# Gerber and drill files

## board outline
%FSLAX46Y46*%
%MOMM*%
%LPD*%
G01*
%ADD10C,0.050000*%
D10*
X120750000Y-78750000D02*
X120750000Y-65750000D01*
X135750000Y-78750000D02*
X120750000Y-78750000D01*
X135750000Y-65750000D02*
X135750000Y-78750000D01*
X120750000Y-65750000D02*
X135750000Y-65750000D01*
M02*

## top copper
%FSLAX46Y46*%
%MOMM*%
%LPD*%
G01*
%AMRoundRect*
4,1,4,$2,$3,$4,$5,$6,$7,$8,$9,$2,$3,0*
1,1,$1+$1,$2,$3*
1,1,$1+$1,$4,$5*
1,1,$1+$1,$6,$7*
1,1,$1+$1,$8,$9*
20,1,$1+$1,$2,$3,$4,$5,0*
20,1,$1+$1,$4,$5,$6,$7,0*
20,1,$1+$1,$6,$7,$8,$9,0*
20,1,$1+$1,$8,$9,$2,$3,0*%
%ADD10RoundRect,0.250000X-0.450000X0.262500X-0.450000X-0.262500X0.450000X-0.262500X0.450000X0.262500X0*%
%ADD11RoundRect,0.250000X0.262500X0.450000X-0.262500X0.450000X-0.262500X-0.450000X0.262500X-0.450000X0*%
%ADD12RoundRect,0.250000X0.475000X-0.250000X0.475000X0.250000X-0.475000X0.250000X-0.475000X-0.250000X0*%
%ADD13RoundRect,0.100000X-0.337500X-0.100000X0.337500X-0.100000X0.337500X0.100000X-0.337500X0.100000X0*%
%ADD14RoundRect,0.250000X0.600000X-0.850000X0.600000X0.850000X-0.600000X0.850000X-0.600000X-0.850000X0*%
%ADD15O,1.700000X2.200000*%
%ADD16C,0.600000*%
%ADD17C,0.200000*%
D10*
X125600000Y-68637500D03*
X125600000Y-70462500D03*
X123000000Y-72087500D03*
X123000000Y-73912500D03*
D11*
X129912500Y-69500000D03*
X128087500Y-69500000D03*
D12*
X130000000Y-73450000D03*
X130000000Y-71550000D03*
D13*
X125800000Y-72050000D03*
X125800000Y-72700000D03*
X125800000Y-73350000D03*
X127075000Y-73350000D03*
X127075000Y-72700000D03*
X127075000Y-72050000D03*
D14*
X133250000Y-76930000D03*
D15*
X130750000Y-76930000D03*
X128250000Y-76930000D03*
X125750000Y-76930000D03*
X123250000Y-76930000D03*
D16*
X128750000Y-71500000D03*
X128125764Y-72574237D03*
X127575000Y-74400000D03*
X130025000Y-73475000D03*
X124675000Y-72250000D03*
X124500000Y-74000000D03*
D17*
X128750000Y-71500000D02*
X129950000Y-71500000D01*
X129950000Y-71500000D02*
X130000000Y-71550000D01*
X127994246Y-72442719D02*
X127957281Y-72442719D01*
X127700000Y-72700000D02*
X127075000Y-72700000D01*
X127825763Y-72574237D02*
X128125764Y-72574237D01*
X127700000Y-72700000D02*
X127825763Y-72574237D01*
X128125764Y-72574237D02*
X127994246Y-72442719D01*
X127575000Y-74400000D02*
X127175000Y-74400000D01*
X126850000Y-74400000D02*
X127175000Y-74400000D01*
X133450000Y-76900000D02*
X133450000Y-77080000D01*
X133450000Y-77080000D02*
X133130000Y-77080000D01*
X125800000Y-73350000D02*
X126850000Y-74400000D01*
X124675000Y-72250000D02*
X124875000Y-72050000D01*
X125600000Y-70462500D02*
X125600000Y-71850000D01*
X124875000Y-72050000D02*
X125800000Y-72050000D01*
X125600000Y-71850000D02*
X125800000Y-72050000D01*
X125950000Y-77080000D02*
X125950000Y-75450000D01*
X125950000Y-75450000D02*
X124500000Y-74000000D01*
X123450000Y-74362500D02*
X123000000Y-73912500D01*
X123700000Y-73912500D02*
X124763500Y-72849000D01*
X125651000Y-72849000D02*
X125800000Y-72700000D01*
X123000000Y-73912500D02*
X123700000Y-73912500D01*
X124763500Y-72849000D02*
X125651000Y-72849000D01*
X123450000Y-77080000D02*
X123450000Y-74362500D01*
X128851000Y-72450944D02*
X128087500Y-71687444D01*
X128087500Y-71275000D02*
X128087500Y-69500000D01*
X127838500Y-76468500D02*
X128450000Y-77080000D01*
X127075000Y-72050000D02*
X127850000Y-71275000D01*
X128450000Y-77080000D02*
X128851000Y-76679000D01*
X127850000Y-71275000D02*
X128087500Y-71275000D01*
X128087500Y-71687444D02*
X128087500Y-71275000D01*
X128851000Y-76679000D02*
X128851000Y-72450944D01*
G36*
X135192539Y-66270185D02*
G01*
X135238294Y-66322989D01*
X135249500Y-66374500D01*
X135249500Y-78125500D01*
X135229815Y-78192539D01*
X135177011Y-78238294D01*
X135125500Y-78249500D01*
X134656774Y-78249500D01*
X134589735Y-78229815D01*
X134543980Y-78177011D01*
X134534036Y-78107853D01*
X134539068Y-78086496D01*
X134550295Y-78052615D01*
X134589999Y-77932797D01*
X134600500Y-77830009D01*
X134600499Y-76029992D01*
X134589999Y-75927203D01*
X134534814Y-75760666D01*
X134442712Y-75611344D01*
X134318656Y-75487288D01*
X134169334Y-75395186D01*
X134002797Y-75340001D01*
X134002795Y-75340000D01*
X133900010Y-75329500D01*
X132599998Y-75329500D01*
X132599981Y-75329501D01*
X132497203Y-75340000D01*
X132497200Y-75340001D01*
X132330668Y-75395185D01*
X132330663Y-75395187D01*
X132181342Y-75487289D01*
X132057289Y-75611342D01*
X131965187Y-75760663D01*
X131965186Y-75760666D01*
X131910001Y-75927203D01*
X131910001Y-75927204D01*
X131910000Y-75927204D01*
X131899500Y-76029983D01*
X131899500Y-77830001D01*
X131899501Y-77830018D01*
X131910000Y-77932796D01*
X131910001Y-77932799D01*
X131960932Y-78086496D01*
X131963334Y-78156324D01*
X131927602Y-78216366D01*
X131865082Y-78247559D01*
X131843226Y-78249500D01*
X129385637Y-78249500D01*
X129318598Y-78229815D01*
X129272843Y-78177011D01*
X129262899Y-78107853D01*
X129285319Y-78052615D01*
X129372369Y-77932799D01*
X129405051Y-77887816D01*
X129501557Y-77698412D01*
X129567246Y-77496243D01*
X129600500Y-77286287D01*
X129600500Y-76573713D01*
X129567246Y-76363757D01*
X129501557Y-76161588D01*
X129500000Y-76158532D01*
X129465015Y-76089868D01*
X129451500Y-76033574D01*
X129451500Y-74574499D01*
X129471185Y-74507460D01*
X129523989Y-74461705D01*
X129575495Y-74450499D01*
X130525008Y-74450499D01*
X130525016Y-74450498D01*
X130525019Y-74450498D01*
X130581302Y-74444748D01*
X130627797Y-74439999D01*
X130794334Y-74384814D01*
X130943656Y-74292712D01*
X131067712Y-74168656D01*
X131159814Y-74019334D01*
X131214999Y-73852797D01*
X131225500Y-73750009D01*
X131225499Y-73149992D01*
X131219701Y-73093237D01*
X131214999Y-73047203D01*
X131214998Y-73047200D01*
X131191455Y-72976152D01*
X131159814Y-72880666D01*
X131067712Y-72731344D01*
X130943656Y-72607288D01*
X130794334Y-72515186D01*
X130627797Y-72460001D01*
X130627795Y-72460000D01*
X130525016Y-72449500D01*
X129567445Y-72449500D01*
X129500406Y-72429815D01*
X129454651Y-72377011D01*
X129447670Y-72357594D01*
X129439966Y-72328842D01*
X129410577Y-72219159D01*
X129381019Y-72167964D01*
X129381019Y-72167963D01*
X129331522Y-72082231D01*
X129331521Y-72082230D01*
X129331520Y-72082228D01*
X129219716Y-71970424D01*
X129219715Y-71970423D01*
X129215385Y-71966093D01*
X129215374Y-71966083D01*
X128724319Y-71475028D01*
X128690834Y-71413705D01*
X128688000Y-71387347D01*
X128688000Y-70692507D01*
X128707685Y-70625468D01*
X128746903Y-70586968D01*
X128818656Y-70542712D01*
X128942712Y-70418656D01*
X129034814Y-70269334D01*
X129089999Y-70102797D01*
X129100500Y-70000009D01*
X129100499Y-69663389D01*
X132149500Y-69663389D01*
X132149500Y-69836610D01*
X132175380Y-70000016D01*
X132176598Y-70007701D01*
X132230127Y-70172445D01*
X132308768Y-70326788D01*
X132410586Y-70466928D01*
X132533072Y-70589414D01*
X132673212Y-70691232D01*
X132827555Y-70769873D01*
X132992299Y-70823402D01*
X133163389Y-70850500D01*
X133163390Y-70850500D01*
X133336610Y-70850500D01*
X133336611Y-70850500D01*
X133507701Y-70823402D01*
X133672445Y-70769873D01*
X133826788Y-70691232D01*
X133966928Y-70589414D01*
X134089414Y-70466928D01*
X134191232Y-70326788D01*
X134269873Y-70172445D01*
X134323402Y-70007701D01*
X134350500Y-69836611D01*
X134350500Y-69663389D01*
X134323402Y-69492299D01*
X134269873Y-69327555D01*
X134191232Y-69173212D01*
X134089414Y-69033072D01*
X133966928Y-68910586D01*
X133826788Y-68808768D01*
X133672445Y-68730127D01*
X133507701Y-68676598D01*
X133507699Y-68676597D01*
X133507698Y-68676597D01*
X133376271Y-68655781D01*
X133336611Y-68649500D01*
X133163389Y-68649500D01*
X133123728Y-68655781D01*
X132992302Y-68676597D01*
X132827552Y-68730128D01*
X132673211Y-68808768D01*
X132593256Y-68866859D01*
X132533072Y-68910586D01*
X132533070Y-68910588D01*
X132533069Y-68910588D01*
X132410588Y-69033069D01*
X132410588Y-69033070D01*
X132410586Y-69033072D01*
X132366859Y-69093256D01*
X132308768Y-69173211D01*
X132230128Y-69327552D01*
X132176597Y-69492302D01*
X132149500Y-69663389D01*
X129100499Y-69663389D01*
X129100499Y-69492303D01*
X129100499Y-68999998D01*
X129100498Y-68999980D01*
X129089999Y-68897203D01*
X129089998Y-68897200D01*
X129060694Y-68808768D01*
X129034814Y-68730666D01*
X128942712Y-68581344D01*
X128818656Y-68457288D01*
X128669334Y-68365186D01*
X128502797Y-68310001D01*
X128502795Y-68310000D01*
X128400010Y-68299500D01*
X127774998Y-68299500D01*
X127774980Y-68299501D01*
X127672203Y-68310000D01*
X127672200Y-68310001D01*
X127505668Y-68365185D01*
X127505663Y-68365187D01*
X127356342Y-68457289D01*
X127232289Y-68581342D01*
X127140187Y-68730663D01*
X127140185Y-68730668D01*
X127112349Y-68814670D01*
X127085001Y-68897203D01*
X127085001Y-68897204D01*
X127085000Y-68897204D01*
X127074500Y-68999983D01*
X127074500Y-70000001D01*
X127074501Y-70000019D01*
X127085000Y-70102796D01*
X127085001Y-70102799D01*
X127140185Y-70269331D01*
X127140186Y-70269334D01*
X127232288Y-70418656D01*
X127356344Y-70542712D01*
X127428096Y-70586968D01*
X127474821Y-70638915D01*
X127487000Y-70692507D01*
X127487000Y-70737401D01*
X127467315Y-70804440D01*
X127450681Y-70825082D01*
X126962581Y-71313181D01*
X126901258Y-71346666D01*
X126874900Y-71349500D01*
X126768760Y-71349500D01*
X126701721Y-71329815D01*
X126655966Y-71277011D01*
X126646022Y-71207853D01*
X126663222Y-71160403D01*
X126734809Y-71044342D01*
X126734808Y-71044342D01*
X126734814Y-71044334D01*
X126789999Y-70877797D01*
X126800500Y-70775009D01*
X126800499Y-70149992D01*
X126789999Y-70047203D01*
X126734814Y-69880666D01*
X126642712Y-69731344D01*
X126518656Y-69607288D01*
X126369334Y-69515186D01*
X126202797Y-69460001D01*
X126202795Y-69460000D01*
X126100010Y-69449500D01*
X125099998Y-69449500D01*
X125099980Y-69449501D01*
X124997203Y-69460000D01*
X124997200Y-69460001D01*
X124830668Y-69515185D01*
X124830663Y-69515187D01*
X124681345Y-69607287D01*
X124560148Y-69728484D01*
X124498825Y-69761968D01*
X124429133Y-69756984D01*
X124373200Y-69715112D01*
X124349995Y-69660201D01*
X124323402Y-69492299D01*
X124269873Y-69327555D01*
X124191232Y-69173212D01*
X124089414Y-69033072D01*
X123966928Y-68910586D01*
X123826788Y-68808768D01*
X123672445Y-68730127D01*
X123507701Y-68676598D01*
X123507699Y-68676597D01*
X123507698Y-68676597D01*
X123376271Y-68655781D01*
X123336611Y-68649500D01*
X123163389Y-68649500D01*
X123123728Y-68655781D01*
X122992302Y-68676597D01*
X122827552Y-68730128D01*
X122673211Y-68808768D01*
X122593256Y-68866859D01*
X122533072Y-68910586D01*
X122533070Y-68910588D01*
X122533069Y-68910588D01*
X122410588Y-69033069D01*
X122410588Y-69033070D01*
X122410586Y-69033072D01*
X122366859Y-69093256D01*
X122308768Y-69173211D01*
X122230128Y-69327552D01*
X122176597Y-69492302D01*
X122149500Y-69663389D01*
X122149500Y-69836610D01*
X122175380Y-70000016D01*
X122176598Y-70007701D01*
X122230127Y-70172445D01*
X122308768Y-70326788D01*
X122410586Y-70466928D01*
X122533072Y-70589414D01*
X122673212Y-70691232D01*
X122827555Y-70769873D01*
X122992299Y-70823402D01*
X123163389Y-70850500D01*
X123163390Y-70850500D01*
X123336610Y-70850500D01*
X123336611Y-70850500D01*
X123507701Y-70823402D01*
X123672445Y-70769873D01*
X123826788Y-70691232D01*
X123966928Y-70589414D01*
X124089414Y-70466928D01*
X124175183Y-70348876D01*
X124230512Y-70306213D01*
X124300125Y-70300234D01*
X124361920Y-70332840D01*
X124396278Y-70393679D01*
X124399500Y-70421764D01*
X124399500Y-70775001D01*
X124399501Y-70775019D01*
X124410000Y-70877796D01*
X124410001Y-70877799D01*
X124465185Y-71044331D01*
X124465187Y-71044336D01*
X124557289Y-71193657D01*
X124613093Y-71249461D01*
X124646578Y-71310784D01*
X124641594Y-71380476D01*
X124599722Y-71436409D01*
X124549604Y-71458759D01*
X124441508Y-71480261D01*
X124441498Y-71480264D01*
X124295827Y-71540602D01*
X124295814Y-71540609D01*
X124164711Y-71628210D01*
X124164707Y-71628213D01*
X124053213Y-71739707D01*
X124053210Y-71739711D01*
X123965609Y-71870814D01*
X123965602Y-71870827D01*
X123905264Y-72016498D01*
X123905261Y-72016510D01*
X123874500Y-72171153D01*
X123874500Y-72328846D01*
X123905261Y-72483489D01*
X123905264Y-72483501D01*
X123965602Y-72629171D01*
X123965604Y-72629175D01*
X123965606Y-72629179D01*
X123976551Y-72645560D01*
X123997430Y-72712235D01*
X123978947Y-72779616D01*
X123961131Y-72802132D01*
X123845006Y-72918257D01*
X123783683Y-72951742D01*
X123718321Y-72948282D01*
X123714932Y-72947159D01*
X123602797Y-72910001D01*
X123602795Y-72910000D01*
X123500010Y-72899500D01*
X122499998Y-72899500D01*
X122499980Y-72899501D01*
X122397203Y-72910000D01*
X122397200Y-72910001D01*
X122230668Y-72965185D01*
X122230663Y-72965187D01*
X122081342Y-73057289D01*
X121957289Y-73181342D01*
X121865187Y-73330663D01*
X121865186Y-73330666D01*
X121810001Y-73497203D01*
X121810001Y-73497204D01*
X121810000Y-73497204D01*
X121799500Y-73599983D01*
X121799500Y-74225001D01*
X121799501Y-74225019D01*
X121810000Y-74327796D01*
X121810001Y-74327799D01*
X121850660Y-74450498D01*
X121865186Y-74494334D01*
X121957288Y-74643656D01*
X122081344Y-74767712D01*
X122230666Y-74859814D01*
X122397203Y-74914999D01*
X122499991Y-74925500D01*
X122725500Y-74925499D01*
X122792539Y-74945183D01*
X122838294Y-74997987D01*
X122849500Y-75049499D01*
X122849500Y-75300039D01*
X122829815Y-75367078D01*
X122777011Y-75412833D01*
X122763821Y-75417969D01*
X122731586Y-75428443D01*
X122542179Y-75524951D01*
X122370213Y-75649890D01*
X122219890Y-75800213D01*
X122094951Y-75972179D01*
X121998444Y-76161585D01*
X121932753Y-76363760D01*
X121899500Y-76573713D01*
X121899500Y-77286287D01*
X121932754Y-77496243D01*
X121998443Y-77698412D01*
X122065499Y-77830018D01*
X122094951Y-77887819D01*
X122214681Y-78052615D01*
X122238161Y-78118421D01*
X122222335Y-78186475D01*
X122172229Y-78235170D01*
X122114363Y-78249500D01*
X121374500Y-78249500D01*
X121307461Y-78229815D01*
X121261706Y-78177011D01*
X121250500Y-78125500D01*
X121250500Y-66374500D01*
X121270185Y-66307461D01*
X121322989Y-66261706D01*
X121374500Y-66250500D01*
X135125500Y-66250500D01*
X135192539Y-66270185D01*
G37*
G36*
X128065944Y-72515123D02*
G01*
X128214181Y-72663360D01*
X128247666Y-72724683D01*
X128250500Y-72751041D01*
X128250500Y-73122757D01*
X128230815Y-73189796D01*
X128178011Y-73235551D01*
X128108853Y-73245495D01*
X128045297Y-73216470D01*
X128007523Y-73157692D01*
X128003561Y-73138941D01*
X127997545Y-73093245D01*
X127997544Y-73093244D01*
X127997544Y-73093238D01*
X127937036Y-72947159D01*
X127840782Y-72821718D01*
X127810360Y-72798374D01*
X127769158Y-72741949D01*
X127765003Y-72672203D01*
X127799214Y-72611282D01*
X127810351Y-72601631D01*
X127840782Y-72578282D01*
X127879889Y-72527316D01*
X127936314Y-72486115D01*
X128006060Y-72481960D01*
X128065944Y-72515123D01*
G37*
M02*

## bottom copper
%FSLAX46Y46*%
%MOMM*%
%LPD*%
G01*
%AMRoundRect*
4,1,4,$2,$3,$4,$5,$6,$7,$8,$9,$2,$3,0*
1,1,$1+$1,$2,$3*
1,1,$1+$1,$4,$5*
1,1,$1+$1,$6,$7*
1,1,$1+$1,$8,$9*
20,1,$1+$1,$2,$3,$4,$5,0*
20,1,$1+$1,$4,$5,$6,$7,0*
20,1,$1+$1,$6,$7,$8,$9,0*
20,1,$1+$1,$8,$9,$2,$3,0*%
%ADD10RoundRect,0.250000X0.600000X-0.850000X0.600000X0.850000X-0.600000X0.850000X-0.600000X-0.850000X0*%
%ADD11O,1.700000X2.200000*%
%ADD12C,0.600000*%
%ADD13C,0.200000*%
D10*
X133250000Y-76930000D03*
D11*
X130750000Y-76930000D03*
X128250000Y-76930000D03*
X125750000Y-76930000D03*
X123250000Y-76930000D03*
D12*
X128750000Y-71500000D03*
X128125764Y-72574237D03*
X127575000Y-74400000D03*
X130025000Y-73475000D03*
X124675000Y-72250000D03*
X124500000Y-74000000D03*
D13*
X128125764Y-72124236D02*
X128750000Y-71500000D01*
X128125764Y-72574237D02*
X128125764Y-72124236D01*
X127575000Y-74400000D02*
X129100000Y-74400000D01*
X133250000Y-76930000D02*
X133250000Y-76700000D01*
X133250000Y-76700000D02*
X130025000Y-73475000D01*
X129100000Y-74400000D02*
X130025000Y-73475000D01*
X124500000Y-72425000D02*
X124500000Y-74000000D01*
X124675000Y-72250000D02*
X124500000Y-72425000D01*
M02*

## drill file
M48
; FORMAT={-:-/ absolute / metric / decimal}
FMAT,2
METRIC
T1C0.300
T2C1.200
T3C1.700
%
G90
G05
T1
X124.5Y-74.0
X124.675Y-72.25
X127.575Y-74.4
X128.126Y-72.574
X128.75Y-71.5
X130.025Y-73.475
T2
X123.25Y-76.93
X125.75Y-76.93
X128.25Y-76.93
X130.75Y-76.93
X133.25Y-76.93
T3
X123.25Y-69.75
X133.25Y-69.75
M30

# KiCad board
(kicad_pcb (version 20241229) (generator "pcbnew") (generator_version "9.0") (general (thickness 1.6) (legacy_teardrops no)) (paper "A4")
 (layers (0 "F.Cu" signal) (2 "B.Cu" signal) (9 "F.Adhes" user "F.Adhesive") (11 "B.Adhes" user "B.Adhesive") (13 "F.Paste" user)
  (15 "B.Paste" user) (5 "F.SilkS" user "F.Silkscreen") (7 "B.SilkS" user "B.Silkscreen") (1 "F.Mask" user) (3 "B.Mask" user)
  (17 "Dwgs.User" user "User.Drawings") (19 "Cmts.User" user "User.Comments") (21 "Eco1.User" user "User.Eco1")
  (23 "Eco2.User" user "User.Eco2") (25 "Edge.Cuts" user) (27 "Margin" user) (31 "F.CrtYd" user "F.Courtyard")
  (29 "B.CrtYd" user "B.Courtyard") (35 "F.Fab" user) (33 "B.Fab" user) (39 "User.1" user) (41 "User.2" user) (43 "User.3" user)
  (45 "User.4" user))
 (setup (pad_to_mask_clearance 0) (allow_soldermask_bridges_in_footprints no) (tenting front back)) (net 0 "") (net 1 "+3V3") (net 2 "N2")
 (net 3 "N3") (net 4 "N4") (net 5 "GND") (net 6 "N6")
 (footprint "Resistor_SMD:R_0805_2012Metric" (layer "F.Cu") (at 125.6 69.55 -90)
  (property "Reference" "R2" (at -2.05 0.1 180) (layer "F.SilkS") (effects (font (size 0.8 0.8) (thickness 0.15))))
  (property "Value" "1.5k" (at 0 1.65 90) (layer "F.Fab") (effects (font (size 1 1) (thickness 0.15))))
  (pad "1" smd roundrect (at -0.9125 0 270) (size 1.025 1.4) (layers "F.Cu" "F.Mask" "F.Paste") (roundrect_rratio 0.243902) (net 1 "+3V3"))
  (pad "2" smd roundrect (at 0.9125 0 270) (size 1.025 1.4) (layers "F.Cu" "F.Mask" "F.Paste") (roundrect_rratio 0.243902) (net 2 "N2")))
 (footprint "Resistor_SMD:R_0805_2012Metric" (layer "F.Cu") (at 123 73 -90)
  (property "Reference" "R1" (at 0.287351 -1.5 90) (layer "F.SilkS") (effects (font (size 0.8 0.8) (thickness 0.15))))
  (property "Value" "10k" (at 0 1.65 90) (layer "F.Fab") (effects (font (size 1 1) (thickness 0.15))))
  (pad "1" smd roundrect (at -0.9125 0 270) (size 1.025 1.4) (layers "F.Cu" "F.Mask" "F.Paste") (roundrect_rratio 0.243902) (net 1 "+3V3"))
  (pad "2" smd roundrect (at 0.9125 0 270) (size 1.025 1.4) (layers "F.Cu" "F.Mask" "F.Paste") (roundrect_rratio 0.243902) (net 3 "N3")))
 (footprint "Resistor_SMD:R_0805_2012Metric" (layer "F.Cu") (at 129 69.5 180)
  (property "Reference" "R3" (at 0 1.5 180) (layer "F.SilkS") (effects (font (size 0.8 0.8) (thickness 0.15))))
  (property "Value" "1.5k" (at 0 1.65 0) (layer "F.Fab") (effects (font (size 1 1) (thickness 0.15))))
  (pad "1" smd roundrect (at -0.9125 0 180) (size 1.025 1.4) (layers "F.Cu" "F.Mask" "F.Paste") (roundrect_rratio 0.243902) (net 1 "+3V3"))
  (pad "2" smd roundrect (at 0.9125 0 180) (size 1.025 1.4) (layers "F.Cu" "F.Mask" "F.Paste") (roundrect_rratio 0.243902) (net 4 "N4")))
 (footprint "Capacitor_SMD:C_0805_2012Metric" (layer "F.Cu") (at 130 72.5 90)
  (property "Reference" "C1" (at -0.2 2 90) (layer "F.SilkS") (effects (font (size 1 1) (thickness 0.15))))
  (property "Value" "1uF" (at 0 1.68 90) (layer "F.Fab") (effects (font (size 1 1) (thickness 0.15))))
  (pad "1" smd roundrect (at -0.95 0 90) (size 1 1.45) (layers "F.Cu" "F.Mask" "F.Paste") (roundrect_rratio 0.25) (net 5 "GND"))
  (pad "2" smd roundrect (at 0.95 0 90) (size 1 1.45) (layers "F.Cu" "F.Mask" "F.Paste") (roundrect_rratio 0.25) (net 1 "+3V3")))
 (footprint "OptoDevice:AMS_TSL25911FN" (layer "F.Cu") (at 126.4375 72.7)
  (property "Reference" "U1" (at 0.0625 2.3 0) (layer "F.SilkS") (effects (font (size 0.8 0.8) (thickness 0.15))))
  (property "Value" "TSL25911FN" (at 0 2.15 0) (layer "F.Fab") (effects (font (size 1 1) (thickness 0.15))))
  (pad "1" smd roundrect (at -0.6375 -0.65) (size 0.875 0.4) (layers "F.Cu" "F.Mask" "F.Paste") (roundrect_rratio 0.25) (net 2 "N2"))
  (pad "2" smd roundrect (at -0.6375 0) (size 0.875 0.4) (layers "F.Cu" "F.Mask" "F.Paste") (roundrect_rratio 0.25) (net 3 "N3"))
  (pad "3" smd roundrect (at -0.6375 0.65) (size 0.875 0.4) (layers "F.Cu" "F.Mask" "F.Paste") (roundrect_rratio 0.25) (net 5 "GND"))
  (pad "4" smd roundrect (at 0.6375 0.65) (size 0.875 0.4) (layers "F.Cu" "F.Mask" "F.Paste") (roundrect_rratio 0.25) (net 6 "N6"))
  (pad "5" smd roundrect (at 0.6375 0) (size 0.875 0.4) (layers "F.Cu" "F.Mask" "F.Paste") (roundrect_rratio 0.25) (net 1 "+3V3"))
  (pad "6" smd roundrect (at 0.6375 -0.65) (size 0.875 0.4) (layers "F.Cu" "F.Mask" "F.Paste") (roundrect_rratio 0.25) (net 4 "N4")))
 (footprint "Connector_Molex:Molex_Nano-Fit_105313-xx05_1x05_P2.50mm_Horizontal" (layer "B.Cu") (at 133.25 76.93 90)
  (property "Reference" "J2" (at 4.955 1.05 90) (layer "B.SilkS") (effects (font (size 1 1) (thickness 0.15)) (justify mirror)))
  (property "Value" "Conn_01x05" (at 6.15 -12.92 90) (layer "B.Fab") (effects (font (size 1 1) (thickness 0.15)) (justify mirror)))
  (pad "" np_thru_hole circle (at 7.18 -10 90) (size 1.7 1.7) (drill 1.7) (layers "*.Cu" "*.Mask"))
  (pad "" np_thru_hole circle (at 7.18 0 90) (size 1.7 1.7) (drill 1.7) (layers "*.Cu" "*.Mask"))
  (pad "1" thru_hole roundrect (at 0 0 90) (size 2.2 1.7) (drill 1.2) (layers "*.Cu" "*.Mask") (remove_unused_layers no)
   (roundrect_rratio 0.147059) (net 5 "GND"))
  (pad "2" thru_hole oval (at 0 -2.5 90) (size 2.2 1.7) (drill 1.2) (layers "*.Cu" "*.Mask") (remove_unused_layers no) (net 1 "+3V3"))
  (pad "3" thru_hole oval (at 0 -5 90) (size 2.2 1.7) (drill 1.2) (layers "*.Cu" "*.Mask") (remove_unused_layers no) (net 4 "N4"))
  (pad "4" thru_hole oval (at 0 -7.5 90) (size 2.2 1.7) (drill 1.2) (layers "*.Cu" "*.Mask") (remove_unused_layers no) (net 2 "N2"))
  (pad "5" thru_hole oval (at 0 -10 90) (size 2.2 1.7) (drill 1.2) (layers "*.Cu" "*.Mask") (remove_unused_layers no) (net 3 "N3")))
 (gr_line (start 120.75 78.75) (end 120.75 65.75) (stroke (width 0.05) (type default)) (layer "Edge.Cuts"))
 (gr_line (start 135.75 78.75) (end 120.75 78.75) (stroke (width 0.05) (type default)) (layer "Edge.Cuts"))
 (gr_line (start 135.75 65.75) (end 135.75 78.75) (stroke (width 0.05) (type default)) (layer "Edge.Cuts"))
 (gr_line (start 120.75 65.75) (end 135.75 65.75) (stroke (width 0.05) (type default)) (layer "Edge.Cuts"))
 (segment (start 128.75 71.5) (end 129.95 71.5) (width 0.2) (layer "F.Cu") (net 1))
 (segment (start 129.95 71.5) (end 130 71.55) (width 0.2) (layer "F.Cu") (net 1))
 (segment (start 127.994246 72.442719) (end 127.957281 72.442719) (width 0.2) (layer "F.Cu") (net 1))
 (segment (start 127.7 72.7) (end 127.075 72.7) (width 0.2) (layer "F.Cu") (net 1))
 (segment (start 127.825763 72.574237) (end 128.125764 72.574237) (width 0.2) (layer "F.Cu") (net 1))
 (segment (start 127.7 72.7) (end 127.825763 72.574237) (width 0.2) (layer "F.Cu") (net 1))
 (segment (start 128.125764 72.574237) (end 127.994246 72.442719) (width 0.2) (layer "F.Cu") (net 1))
 (via (at 128.75 71.5) (size 0.6) (drill 0.3) (layers "F.Cu" "B.Cu") (free yes) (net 1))
 (via (at 128.125764 72.574237) (size 0.6) (drill 0.3) (layers "F.Cu" "B.Cu") (free yes) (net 1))
 (segment (start 128.125764 72.124236) (end 128.75 71.5) (width 0.2) (layer "B.Cu") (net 1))
 (segment (start 128.125764 72.574237) (end 128.125764 72.124236) (width 0.2) (layer "B.Cu") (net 1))
 (segment (start 127.575 74.4) (end 127.175 74.4) (width 0.2) (layer "F.Cu") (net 5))
 (segment (start 126.85 74.4) (end 127.175 74.4) (width 0.2) (layer "F.Cu") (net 5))
 (segment (start 133.45 76.9) (end 133.45 77.08) (width 0.2) (layer "F.Cu") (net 5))
 (segment (start 133.45 77.08) (end 133.13 77.08) (width 0.2) (layer "F.Cu") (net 5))
 (segment (start 125.8 73.35) (end 126.85 74.4) (width 0.2) (layer "F.Cu") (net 5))
 (via (at 127.575 74.4) (size 0.6) (drill 0.3) (layers "F.Cu" "B.Cu") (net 5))
 (via (at 130.025 73.475) (size 0.6) (drill 0.3) (layers "F.Cu" "B.Cu") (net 5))
 (segment (start 127.575 74.4) (end 129.1 74.4) (width 0.2) (layer "B.Cu") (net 5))
 (segment (start 133.25 76.93) (end 133.25 76.7) (width 0.2) (layer "B.Cu") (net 5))
 (segment (start 133.25 76.7) (end 130.025 73.475) (width 0.2) (layer "B.Cu") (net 5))
 (segment (start 129.1 74.4) (end 130.025 73.475) (width 0.2) (layer "B.Cu") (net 5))
 (segment (start 124.675 72.25) (end 124.875 72.05) (width 0.2) (layer "F.Cu") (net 2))
 (segment (start 125.6 70.4625) (end 125.6 71.85) (width 0.2) (layer "F.Cu") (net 2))
 (segment (start 124.875 72.05) (end 125.8 72.05) (width 0.2) (layer "F.Cu") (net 2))
 (segment (start 125.6 71.85) (end 125.8 72.05) (width 0.2) (layer "F.Cu") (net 2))
 (segment (start 125.95 77.08) (end 125.95 75.45) (width 0.2) (layer "F.Cu") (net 2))
 (segment (start 125.95 75.45) (end 124.5 74) (width 0.2) (layer "F.Cu") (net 2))
 (via (at 124.675 72.25) (size 0.6) (drill 0.3) (layers "F.Cu" "B.Cu") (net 2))
 (via (at 124.5 74) (size 0.6) (drill 0.3) (layers "F.Cu" "B.Cu") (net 2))
 (segment (start 124.5 72.425) (end 124.5 74) (width 0.2) (layer "B.Cu") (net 2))
 (segment (start 124.675 72.25) (end 124.5 72.425) (width 0.2) (layer "B.Cu") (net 2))
 (segment (start 123.45 74.3625) (end 123 73.9125) (width 0.2) (layer "F.Cu") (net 3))
 (segment (start 123.7 73.9125) (end 124.7635 72.849) (width 0.2) (layer "F.Cu") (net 3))
 (segment (start 125.651 72.849) (end 125.8 72.7) (width 0.2) (layer "F.Cu") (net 3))
 (segment (start 123 73.9125) (end 123.7 73.9125) (width 0.2) (layer "F.Cu") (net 3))
 (segment (start 124.7635 72.849) (end 125.651 72.849) (width 0.2) (layer "F.Cu") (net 3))
 (segment (start 123.45 77.08) (end 123.45 74.3625) (width 0.2) (layer "F.Cu") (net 3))
 (segment (start 128.851 72.450944) (end 128.0875 71.687444) (width 0.2) (layer "F.Cu") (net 4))
 (segment (start 128.0875 71.275) (end 128.0875 69.5) (width 0.2) (layer "F.Cu") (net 4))
 (segment (start 127.8385 76.4685) (end 128.45 77.08) (width 0.2) (layer "F.Cu") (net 4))
 (segment (start 127.075 72.05) (end 127.85 71.275) (width 0.2) (layer "F.Cu") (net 4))
 (segment (start 128.45 77.08) (end 128.851 76.679) (width 0.2) (layer "F.Cu") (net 4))
 (segment (start 127.85 71.275) (end 128.0875 71.275) (width 0.2) (layer "F.Cu") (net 4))
 (segment (start 128.0875 71.687444) (end 128.0875 71.275) (width 0.2) (layer "F.Cu") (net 4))
 (segment (start 128.851 76.679) (end 128.851 72.450944) (width 0.2) (layer "F.Cu") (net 4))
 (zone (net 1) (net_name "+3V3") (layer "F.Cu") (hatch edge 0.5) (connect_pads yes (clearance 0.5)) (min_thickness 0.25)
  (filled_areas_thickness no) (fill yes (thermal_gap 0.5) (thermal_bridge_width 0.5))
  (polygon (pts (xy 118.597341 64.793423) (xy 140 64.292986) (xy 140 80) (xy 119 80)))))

